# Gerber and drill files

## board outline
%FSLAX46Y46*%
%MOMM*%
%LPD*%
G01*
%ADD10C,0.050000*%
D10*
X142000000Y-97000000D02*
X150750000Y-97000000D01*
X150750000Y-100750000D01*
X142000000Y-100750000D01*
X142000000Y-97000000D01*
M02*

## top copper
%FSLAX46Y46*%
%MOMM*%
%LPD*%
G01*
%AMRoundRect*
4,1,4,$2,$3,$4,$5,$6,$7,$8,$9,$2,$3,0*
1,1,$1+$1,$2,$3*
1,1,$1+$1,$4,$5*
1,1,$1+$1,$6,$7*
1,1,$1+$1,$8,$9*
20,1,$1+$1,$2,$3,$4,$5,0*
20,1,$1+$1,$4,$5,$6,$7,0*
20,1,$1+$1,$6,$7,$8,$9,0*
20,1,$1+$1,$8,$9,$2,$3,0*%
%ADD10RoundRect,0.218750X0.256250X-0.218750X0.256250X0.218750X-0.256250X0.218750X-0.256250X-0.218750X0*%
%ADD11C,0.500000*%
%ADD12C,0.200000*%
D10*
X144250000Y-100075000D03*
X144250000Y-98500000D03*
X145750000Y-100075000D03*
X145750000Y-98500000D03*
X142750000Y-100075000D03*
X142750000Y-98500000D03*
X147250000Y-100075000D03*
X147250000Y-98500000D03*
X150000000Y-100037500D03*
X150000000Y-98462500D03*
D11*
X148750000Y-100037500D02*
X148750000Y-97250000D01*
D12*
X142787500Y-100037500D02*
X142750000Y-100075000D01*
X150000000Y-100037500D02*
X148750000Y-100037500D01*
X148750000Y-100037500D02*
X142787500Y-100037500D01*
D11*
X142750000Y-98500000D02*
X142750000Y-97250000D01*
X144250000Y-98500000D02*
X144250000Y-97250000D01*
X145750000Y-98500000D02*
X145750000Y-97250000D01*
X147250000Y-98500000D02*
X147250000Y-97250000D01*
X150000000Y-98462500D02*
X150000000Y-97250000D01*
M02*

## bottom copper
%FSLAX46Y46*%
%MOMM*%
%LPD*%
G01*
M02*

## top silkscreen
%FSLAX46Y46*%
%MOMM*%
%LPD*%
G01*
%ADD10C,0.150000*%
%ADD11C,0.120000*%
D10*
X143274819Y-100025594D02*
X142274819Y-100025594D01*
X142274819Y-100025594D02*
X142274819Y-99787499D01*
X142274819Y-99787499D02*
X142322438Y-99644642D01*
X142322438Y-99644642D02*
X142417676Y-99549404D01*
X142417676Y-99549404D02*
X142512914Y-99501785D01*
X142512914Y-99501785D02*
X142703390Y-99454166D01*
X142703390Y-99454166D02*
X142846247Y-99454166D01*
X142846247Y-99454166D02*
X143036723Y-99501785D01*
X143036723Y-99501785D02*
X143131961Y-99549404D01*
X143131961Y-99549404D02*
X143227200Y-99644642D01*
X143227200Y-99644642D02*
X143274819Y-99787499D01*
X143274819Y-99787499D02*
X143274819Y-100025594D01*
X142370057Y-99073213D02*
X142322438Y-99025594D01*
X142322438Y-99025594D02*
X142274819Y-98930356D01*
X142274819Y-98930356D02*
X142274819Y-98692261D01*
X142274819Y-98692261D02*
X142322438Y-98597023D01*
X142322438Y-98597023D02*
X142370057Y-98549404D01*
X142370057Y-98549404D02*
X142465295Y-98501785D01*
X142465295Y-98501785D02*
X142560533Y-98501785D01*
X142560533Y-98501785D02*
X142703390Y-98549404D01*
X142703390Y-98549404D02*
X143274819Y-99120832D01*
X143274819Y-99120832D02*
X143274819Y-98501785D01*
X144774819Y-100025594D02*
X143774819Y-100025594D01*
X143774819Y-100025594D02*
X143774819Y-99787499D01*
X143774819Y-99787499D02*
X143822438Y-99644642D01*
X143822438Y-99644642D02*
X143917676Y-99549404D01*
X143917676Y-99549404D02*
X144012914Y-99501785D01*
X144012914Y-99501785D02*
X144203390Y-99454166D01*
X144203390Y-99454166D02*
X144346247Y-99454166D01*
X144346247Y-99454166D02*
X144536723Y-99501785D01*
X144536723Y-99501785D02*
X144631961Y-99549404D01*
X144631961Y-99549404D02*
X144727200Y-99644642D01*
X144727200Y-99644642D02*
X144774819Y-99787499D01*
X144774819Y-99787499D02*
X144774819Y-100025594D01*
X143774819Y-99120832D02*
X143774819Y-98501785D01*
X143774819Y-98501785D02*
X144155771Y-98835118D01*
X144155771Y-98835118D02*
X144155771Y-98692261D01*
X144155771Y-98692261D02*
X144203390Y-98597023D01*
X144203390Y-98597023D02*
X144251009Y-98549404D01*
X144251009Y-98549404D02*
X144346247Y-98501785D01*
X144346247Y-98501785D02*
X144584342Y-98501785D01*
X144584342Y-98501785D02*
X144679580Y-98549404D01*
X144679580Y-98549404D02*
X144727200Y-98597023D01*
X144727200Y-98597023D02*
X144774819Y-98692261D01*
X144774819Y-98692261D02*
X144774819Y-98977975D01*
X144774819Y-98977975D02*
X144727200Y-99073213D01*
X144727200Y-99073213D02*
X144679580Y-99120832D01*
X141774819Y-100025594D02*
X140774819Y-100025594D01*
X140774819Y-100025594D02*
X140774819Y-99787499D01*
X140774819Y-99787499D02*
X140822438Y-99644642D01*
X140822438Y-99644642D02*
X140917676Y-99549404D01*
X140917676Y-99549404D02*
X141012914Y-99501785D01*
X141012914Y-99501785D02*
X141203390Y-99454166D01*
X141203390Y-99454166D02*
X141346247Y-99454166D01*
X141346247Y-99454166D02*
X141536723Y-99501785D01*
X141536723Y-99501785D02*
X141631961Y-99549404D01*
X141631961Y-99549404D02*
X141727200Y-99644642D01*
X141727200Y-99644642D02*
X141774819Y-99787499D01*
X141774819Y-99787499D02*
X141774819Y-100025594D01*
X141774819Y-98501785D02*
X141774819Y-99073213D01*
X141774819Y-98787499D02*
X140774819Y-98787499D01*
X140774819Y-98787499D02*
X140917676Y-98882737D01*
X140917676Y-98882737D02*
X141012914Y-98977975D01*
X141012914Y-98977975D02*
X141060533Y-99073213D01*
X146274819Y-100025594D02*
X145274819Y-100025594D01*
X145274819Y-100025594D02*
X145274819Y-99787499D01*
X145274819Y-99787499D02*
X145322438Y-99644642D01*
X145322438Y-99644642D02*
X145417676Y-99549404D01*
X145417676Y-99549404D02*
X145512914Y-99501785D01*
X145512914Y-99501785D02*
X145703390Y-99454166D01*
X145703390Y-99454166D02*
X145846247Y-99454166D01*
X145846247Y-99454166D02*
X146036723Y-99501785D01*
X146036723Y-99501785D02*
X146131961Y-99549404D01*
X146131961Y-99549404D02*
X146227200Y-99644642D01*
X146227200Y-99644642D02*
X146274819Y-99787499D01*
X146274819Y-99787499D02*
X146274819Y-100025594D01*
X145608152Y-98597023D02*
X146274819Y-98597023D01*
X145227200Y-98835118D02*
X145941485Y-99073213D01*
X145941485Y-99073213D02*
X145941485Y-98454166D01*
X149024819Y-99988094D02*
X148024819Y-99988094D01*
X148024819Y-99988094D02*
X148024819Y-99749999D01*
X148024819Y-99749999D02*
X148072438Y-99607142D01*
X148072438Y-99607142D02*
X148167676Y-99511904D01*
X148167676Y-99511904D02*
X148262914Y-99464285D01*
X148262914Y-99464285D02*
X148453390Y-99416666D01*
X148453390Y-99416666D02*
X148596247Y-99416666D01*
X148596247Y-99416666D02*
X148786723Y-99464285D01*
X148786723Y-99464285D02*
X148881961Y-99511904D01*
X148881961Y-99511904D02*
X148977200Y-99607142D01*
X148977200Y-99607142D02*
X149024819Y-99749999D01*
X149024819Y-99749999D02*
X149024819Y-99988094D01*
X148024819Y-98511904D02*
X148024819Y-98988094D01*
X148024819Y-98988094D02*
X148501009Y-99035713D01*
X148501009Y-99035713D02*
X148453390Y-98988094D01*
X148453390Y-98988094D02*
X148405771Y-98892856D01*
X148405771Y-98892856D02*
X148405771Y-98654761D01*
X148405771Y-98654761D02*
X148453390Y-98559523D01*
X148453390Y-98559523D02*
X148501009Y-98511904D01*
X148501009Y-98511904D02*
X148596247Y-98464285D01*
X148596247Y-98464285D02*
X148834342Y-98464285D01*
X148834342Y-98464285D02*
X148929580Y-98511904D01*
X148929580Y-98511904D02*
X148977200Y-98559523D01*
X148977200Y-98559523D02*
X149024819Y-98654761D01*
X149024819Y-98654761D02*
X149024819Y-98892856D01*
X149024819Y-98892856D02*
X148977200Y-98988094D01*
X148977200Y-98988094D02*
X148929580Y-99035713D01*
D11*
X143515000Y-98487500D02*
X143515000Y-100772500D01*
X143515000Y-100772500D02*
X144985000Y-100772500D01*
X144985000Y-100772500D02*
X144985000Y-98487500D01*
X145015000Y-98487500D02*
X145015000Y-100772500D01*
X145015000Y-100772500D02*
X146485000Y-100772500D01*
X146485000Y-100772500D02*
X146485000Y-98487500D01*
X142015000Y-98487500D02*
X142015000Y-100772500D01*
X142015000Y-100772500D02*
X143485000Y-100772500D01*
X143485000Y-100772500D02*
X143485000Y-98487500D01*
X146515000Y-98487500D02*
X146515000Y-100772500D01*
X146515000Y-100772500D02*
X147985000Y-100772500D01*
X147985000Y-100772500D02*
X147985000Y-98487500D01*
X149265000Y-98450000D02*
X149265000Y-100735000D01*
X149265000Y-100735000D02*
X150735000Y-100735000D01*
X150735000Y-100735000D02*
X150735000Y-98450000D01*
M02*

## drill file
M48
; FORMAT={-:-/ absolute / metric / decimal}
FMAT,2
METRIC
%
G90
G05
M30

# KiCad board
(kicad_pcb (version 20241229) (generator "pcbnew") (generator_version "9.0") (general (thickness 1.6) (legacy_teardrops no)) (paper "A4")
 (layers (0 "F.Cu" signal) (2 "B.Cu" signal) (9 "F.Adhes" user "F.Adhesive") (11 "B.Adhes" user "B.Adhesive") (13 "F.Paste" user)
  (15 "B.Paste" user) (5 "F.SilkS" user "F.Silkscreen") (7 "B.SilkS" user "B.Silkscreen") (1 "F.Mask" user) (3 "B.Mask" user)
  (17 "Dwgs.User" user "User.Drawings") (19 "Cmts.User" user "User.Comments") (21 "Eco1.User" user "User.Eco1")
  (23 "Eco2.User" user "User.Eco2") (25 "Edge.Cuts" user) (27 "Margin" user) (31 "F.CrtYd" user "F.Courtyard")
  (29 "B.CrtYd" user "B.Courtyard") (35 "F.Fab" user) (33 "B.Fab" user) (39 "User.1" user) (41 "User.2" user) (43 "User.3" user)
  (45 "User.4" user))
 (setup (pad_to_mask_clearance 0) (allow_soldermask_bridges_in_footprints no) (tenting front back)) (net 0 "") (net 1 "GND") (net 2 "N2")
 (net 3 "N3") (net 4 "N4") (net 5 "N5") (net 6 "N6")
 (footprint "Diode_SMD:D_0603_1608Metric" (layer "F.Cu") (at 144.25 99.2875 90)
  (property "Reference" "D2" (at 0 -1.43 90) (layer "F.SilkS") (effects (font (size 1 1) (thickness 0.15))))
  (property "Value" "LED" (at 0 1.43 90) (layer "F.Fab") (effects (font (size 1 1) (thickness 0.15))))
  (fp_line (start 0.8 -0.735) (end -1.485 -0.735) (stroke (width 0.12) (type solid)) (layer "F.SilkS"))
  (fp_line (start -1.485 -0.735) (end -1.485 0.735) (stroke (width 0.12) (type solid)) (layer "F.SilkS"))
  (fp_line (start -1.485 0.735) (end 0.8 0.735) (stroke (width 0.12) (type solid)) (layer "F.SilkS"))
  (pad "1" smd roundrect (at -0.7875 0 90) (size 0.875 0.95) (layers "F.Cu" "F.Mask" "F.Paste") (roundrect_rratio 0.25) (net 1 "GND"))
  (pad "2" smd roundrect (at 0.7875 0 90) (size 0.875 0.95) (layers "F.Cu" "F.Mask" "F.Paste") (roundrect_rratio 0.25) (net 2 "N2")))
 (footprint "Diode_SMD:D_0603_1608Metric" (layer "F.Cu") (at 145.75 99.2875 90)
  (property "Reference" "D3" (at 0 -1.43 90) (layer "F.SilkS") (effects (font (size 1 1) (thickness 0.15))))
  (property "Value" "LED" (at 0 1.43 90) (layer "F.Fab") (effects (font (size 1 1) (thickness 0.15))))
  (fp_line (start 0.8 -0.735) (end -1.485 -0.735) (stroke (width 0.12) (type solid)) (layer "F.SilkS"))
  (fp_line (start -1.485 -0.735) (end -1.485 0.735) (stroke (width 0.12) (type solid)) (layer "F.SilkS"))
  (fp_line (start -1.485 0.735) (end 0.8 0.735) (stroke (width 0.12) (type solid)) (layer "F.SilkS"))
  (pad "1" smd roundrect (at -0.7875 0 90) (size 0.875 0.95) (layers "F.Cu" "F.Mask" "F.Paste") (roundrect_rratio 0.25) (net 1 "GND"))
  (pad "2" smd roundrect (at 0.7875 0 90) (size 0.875 0.95) (layers "F.Cu" "F.Mask" "F.Paste") (roundrect_rratio 0.25) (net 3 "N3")))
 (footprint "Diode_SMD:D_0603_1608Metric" (layer "F.Cu") (at 142.75 99.2875 90)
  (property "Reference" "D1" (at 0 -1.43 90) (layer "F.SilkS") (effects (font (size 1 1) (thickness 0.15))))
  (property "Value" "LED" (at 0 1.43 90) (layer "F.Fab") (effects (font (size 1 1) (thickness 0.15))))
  (fp_line (start 0.8 -0.735) (end -1.485 -0.735) (stroke (width 0.12) (type solid)) (layer "F.SilkS"))
  (fp_line (start -1.485 -0.735) (end -1.485 0.735) (stroke (width 0.12) (type solid)) (layer "F.SilkS"))
  (fp_line (start -1.485 0.735) (end 0.8 0.735) (stroke (width 0.12) (type solid)) (layer "F.SilkS"))
  (pad "1" smd roundrect (at -0.7875 0 90) (size 0.875 0.95) (layers "F.Cu" "F.Mask" "F.Paste") (roundrect_rratio 0.25) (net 1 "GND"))
  (pad "2" smd roundrect (at 0.7875 0 90) (size 0.875 0.95) (layers "F.Cu" "F.Mask" "F.Paste") (roundrect_rratio 0.25) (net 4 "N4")))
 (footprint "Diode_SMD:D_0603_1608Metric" (layer "F.Cu") (at 147.25 99.2875 90)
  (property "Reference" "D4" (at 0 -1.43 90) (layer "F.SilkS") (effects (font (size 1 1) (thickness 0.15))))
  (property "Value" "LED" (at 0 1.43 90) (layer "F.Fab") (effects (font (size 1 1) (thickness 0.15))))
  (fp_line (start 0.8 -0.735) (end -1.485 -0.735) (stroke (width 0.12) (type solid)) (layer "F.SilkS"))
  (fp_line (start -1.485 -0.735) (end -1.485 0.735) (stroke (width 0.12) (type solid)) (layer "F.SilkS"))
  (fp_line (start -1.485 0.735) (end 0.8 0.735) (stroke (width 0.12) (type solid)) (layer "F.SilkS"))
  (pad "1" smd roundrect (at -0.7875 0 90) (size 0.875 0.95) (layers "F.Cu" "F.Mask" "F.Paste") (roundrect_rratio 0.25) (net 1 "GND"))
  (pad "2" smd roundrect (at 0.7875 0 90) (size 0.875 0.95) (layers "F.Cu" "F.Mask" "F.Paste") (roundrect_rratio 0.25) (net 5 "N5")))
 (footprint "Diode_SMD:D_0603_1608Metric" (layer "F.Cu") (at 150 99.25 90)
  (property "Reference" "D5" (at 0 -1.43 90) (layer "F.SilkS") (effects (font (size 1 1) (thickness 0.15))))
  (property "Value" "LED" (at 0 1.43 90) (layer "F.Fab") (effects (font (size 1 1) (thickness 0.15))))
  (fp_line (start 0.8 -0.735) (end -1.485 -0.735) (stroke (width 0.12) (type solid)) (layer "F.SilkS"))
  (fp_line (start -1.485 -0.735) (end -1.485 0.735) (stroke (width 0.12) (type solid)) (layer "F.SilkS"))
  (fp_line (start -1.485 0.735) (end 0.8 0.735) (stroke (width 0.12) (type solid)) (layer "F.SilkS"))
  (pad "1" smd roundrect (at -0.7875 0 90) (size 0.875 0.95) (layers "F.Cu" "F.Mask" "F.Paste") (roundrect_rratio 0.25) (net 1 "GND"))
  (pad "2" smd roundrect (at 0.7875 0 90) (size 0.875 0.95) (layers "F.Cu" "F.Mask" "F.Paste") (roundrect_rratio 0.25) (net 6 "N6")))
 (gr_rect (start 142 97) (end 150.75 100.75) (stroke (width 0.05) (type default)) (fill no) (layer "Edge.Cuts"))
 (segment (start 148.75 100.0375) (end 148.75 97.25) (width 0.5) (layer "F.Cu") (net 1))
 (segment (start 142.7875 100.0375) (end 142.75 100.075) (width 0.2) (layer "F.Cu") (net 1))
 (segment (start 150 100.0375) (end 148.75 100.0375) (width 0.2) (layer "F.Cu") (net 1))
 (segment (start 148.75 100.0375) (end 142.7875 100.0375) (width 0.2) (layer "F.Cu") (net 1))
 (segment (start 142.75 98.5) (end 142.75 97.25) (width 0.5) (layer "F.Cu") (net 4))
 (segment (start 144.25 98.5) (end 144.25 97.25) (width 0.5) (layer "F.Cu") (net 2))
 (segment (start 145.75 98.5) (end 145.75 97.25) (width 0.5) (layer "F.Cu") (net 3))
 (segment (start 147.25 98.5) (end 147.25 97.25) (width 0.5) (layer "F.Cu") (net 5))
 (segment (start 150 98.4625) (end 150 97.25) (width 0.5) (layer "F.Cu") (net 6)))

